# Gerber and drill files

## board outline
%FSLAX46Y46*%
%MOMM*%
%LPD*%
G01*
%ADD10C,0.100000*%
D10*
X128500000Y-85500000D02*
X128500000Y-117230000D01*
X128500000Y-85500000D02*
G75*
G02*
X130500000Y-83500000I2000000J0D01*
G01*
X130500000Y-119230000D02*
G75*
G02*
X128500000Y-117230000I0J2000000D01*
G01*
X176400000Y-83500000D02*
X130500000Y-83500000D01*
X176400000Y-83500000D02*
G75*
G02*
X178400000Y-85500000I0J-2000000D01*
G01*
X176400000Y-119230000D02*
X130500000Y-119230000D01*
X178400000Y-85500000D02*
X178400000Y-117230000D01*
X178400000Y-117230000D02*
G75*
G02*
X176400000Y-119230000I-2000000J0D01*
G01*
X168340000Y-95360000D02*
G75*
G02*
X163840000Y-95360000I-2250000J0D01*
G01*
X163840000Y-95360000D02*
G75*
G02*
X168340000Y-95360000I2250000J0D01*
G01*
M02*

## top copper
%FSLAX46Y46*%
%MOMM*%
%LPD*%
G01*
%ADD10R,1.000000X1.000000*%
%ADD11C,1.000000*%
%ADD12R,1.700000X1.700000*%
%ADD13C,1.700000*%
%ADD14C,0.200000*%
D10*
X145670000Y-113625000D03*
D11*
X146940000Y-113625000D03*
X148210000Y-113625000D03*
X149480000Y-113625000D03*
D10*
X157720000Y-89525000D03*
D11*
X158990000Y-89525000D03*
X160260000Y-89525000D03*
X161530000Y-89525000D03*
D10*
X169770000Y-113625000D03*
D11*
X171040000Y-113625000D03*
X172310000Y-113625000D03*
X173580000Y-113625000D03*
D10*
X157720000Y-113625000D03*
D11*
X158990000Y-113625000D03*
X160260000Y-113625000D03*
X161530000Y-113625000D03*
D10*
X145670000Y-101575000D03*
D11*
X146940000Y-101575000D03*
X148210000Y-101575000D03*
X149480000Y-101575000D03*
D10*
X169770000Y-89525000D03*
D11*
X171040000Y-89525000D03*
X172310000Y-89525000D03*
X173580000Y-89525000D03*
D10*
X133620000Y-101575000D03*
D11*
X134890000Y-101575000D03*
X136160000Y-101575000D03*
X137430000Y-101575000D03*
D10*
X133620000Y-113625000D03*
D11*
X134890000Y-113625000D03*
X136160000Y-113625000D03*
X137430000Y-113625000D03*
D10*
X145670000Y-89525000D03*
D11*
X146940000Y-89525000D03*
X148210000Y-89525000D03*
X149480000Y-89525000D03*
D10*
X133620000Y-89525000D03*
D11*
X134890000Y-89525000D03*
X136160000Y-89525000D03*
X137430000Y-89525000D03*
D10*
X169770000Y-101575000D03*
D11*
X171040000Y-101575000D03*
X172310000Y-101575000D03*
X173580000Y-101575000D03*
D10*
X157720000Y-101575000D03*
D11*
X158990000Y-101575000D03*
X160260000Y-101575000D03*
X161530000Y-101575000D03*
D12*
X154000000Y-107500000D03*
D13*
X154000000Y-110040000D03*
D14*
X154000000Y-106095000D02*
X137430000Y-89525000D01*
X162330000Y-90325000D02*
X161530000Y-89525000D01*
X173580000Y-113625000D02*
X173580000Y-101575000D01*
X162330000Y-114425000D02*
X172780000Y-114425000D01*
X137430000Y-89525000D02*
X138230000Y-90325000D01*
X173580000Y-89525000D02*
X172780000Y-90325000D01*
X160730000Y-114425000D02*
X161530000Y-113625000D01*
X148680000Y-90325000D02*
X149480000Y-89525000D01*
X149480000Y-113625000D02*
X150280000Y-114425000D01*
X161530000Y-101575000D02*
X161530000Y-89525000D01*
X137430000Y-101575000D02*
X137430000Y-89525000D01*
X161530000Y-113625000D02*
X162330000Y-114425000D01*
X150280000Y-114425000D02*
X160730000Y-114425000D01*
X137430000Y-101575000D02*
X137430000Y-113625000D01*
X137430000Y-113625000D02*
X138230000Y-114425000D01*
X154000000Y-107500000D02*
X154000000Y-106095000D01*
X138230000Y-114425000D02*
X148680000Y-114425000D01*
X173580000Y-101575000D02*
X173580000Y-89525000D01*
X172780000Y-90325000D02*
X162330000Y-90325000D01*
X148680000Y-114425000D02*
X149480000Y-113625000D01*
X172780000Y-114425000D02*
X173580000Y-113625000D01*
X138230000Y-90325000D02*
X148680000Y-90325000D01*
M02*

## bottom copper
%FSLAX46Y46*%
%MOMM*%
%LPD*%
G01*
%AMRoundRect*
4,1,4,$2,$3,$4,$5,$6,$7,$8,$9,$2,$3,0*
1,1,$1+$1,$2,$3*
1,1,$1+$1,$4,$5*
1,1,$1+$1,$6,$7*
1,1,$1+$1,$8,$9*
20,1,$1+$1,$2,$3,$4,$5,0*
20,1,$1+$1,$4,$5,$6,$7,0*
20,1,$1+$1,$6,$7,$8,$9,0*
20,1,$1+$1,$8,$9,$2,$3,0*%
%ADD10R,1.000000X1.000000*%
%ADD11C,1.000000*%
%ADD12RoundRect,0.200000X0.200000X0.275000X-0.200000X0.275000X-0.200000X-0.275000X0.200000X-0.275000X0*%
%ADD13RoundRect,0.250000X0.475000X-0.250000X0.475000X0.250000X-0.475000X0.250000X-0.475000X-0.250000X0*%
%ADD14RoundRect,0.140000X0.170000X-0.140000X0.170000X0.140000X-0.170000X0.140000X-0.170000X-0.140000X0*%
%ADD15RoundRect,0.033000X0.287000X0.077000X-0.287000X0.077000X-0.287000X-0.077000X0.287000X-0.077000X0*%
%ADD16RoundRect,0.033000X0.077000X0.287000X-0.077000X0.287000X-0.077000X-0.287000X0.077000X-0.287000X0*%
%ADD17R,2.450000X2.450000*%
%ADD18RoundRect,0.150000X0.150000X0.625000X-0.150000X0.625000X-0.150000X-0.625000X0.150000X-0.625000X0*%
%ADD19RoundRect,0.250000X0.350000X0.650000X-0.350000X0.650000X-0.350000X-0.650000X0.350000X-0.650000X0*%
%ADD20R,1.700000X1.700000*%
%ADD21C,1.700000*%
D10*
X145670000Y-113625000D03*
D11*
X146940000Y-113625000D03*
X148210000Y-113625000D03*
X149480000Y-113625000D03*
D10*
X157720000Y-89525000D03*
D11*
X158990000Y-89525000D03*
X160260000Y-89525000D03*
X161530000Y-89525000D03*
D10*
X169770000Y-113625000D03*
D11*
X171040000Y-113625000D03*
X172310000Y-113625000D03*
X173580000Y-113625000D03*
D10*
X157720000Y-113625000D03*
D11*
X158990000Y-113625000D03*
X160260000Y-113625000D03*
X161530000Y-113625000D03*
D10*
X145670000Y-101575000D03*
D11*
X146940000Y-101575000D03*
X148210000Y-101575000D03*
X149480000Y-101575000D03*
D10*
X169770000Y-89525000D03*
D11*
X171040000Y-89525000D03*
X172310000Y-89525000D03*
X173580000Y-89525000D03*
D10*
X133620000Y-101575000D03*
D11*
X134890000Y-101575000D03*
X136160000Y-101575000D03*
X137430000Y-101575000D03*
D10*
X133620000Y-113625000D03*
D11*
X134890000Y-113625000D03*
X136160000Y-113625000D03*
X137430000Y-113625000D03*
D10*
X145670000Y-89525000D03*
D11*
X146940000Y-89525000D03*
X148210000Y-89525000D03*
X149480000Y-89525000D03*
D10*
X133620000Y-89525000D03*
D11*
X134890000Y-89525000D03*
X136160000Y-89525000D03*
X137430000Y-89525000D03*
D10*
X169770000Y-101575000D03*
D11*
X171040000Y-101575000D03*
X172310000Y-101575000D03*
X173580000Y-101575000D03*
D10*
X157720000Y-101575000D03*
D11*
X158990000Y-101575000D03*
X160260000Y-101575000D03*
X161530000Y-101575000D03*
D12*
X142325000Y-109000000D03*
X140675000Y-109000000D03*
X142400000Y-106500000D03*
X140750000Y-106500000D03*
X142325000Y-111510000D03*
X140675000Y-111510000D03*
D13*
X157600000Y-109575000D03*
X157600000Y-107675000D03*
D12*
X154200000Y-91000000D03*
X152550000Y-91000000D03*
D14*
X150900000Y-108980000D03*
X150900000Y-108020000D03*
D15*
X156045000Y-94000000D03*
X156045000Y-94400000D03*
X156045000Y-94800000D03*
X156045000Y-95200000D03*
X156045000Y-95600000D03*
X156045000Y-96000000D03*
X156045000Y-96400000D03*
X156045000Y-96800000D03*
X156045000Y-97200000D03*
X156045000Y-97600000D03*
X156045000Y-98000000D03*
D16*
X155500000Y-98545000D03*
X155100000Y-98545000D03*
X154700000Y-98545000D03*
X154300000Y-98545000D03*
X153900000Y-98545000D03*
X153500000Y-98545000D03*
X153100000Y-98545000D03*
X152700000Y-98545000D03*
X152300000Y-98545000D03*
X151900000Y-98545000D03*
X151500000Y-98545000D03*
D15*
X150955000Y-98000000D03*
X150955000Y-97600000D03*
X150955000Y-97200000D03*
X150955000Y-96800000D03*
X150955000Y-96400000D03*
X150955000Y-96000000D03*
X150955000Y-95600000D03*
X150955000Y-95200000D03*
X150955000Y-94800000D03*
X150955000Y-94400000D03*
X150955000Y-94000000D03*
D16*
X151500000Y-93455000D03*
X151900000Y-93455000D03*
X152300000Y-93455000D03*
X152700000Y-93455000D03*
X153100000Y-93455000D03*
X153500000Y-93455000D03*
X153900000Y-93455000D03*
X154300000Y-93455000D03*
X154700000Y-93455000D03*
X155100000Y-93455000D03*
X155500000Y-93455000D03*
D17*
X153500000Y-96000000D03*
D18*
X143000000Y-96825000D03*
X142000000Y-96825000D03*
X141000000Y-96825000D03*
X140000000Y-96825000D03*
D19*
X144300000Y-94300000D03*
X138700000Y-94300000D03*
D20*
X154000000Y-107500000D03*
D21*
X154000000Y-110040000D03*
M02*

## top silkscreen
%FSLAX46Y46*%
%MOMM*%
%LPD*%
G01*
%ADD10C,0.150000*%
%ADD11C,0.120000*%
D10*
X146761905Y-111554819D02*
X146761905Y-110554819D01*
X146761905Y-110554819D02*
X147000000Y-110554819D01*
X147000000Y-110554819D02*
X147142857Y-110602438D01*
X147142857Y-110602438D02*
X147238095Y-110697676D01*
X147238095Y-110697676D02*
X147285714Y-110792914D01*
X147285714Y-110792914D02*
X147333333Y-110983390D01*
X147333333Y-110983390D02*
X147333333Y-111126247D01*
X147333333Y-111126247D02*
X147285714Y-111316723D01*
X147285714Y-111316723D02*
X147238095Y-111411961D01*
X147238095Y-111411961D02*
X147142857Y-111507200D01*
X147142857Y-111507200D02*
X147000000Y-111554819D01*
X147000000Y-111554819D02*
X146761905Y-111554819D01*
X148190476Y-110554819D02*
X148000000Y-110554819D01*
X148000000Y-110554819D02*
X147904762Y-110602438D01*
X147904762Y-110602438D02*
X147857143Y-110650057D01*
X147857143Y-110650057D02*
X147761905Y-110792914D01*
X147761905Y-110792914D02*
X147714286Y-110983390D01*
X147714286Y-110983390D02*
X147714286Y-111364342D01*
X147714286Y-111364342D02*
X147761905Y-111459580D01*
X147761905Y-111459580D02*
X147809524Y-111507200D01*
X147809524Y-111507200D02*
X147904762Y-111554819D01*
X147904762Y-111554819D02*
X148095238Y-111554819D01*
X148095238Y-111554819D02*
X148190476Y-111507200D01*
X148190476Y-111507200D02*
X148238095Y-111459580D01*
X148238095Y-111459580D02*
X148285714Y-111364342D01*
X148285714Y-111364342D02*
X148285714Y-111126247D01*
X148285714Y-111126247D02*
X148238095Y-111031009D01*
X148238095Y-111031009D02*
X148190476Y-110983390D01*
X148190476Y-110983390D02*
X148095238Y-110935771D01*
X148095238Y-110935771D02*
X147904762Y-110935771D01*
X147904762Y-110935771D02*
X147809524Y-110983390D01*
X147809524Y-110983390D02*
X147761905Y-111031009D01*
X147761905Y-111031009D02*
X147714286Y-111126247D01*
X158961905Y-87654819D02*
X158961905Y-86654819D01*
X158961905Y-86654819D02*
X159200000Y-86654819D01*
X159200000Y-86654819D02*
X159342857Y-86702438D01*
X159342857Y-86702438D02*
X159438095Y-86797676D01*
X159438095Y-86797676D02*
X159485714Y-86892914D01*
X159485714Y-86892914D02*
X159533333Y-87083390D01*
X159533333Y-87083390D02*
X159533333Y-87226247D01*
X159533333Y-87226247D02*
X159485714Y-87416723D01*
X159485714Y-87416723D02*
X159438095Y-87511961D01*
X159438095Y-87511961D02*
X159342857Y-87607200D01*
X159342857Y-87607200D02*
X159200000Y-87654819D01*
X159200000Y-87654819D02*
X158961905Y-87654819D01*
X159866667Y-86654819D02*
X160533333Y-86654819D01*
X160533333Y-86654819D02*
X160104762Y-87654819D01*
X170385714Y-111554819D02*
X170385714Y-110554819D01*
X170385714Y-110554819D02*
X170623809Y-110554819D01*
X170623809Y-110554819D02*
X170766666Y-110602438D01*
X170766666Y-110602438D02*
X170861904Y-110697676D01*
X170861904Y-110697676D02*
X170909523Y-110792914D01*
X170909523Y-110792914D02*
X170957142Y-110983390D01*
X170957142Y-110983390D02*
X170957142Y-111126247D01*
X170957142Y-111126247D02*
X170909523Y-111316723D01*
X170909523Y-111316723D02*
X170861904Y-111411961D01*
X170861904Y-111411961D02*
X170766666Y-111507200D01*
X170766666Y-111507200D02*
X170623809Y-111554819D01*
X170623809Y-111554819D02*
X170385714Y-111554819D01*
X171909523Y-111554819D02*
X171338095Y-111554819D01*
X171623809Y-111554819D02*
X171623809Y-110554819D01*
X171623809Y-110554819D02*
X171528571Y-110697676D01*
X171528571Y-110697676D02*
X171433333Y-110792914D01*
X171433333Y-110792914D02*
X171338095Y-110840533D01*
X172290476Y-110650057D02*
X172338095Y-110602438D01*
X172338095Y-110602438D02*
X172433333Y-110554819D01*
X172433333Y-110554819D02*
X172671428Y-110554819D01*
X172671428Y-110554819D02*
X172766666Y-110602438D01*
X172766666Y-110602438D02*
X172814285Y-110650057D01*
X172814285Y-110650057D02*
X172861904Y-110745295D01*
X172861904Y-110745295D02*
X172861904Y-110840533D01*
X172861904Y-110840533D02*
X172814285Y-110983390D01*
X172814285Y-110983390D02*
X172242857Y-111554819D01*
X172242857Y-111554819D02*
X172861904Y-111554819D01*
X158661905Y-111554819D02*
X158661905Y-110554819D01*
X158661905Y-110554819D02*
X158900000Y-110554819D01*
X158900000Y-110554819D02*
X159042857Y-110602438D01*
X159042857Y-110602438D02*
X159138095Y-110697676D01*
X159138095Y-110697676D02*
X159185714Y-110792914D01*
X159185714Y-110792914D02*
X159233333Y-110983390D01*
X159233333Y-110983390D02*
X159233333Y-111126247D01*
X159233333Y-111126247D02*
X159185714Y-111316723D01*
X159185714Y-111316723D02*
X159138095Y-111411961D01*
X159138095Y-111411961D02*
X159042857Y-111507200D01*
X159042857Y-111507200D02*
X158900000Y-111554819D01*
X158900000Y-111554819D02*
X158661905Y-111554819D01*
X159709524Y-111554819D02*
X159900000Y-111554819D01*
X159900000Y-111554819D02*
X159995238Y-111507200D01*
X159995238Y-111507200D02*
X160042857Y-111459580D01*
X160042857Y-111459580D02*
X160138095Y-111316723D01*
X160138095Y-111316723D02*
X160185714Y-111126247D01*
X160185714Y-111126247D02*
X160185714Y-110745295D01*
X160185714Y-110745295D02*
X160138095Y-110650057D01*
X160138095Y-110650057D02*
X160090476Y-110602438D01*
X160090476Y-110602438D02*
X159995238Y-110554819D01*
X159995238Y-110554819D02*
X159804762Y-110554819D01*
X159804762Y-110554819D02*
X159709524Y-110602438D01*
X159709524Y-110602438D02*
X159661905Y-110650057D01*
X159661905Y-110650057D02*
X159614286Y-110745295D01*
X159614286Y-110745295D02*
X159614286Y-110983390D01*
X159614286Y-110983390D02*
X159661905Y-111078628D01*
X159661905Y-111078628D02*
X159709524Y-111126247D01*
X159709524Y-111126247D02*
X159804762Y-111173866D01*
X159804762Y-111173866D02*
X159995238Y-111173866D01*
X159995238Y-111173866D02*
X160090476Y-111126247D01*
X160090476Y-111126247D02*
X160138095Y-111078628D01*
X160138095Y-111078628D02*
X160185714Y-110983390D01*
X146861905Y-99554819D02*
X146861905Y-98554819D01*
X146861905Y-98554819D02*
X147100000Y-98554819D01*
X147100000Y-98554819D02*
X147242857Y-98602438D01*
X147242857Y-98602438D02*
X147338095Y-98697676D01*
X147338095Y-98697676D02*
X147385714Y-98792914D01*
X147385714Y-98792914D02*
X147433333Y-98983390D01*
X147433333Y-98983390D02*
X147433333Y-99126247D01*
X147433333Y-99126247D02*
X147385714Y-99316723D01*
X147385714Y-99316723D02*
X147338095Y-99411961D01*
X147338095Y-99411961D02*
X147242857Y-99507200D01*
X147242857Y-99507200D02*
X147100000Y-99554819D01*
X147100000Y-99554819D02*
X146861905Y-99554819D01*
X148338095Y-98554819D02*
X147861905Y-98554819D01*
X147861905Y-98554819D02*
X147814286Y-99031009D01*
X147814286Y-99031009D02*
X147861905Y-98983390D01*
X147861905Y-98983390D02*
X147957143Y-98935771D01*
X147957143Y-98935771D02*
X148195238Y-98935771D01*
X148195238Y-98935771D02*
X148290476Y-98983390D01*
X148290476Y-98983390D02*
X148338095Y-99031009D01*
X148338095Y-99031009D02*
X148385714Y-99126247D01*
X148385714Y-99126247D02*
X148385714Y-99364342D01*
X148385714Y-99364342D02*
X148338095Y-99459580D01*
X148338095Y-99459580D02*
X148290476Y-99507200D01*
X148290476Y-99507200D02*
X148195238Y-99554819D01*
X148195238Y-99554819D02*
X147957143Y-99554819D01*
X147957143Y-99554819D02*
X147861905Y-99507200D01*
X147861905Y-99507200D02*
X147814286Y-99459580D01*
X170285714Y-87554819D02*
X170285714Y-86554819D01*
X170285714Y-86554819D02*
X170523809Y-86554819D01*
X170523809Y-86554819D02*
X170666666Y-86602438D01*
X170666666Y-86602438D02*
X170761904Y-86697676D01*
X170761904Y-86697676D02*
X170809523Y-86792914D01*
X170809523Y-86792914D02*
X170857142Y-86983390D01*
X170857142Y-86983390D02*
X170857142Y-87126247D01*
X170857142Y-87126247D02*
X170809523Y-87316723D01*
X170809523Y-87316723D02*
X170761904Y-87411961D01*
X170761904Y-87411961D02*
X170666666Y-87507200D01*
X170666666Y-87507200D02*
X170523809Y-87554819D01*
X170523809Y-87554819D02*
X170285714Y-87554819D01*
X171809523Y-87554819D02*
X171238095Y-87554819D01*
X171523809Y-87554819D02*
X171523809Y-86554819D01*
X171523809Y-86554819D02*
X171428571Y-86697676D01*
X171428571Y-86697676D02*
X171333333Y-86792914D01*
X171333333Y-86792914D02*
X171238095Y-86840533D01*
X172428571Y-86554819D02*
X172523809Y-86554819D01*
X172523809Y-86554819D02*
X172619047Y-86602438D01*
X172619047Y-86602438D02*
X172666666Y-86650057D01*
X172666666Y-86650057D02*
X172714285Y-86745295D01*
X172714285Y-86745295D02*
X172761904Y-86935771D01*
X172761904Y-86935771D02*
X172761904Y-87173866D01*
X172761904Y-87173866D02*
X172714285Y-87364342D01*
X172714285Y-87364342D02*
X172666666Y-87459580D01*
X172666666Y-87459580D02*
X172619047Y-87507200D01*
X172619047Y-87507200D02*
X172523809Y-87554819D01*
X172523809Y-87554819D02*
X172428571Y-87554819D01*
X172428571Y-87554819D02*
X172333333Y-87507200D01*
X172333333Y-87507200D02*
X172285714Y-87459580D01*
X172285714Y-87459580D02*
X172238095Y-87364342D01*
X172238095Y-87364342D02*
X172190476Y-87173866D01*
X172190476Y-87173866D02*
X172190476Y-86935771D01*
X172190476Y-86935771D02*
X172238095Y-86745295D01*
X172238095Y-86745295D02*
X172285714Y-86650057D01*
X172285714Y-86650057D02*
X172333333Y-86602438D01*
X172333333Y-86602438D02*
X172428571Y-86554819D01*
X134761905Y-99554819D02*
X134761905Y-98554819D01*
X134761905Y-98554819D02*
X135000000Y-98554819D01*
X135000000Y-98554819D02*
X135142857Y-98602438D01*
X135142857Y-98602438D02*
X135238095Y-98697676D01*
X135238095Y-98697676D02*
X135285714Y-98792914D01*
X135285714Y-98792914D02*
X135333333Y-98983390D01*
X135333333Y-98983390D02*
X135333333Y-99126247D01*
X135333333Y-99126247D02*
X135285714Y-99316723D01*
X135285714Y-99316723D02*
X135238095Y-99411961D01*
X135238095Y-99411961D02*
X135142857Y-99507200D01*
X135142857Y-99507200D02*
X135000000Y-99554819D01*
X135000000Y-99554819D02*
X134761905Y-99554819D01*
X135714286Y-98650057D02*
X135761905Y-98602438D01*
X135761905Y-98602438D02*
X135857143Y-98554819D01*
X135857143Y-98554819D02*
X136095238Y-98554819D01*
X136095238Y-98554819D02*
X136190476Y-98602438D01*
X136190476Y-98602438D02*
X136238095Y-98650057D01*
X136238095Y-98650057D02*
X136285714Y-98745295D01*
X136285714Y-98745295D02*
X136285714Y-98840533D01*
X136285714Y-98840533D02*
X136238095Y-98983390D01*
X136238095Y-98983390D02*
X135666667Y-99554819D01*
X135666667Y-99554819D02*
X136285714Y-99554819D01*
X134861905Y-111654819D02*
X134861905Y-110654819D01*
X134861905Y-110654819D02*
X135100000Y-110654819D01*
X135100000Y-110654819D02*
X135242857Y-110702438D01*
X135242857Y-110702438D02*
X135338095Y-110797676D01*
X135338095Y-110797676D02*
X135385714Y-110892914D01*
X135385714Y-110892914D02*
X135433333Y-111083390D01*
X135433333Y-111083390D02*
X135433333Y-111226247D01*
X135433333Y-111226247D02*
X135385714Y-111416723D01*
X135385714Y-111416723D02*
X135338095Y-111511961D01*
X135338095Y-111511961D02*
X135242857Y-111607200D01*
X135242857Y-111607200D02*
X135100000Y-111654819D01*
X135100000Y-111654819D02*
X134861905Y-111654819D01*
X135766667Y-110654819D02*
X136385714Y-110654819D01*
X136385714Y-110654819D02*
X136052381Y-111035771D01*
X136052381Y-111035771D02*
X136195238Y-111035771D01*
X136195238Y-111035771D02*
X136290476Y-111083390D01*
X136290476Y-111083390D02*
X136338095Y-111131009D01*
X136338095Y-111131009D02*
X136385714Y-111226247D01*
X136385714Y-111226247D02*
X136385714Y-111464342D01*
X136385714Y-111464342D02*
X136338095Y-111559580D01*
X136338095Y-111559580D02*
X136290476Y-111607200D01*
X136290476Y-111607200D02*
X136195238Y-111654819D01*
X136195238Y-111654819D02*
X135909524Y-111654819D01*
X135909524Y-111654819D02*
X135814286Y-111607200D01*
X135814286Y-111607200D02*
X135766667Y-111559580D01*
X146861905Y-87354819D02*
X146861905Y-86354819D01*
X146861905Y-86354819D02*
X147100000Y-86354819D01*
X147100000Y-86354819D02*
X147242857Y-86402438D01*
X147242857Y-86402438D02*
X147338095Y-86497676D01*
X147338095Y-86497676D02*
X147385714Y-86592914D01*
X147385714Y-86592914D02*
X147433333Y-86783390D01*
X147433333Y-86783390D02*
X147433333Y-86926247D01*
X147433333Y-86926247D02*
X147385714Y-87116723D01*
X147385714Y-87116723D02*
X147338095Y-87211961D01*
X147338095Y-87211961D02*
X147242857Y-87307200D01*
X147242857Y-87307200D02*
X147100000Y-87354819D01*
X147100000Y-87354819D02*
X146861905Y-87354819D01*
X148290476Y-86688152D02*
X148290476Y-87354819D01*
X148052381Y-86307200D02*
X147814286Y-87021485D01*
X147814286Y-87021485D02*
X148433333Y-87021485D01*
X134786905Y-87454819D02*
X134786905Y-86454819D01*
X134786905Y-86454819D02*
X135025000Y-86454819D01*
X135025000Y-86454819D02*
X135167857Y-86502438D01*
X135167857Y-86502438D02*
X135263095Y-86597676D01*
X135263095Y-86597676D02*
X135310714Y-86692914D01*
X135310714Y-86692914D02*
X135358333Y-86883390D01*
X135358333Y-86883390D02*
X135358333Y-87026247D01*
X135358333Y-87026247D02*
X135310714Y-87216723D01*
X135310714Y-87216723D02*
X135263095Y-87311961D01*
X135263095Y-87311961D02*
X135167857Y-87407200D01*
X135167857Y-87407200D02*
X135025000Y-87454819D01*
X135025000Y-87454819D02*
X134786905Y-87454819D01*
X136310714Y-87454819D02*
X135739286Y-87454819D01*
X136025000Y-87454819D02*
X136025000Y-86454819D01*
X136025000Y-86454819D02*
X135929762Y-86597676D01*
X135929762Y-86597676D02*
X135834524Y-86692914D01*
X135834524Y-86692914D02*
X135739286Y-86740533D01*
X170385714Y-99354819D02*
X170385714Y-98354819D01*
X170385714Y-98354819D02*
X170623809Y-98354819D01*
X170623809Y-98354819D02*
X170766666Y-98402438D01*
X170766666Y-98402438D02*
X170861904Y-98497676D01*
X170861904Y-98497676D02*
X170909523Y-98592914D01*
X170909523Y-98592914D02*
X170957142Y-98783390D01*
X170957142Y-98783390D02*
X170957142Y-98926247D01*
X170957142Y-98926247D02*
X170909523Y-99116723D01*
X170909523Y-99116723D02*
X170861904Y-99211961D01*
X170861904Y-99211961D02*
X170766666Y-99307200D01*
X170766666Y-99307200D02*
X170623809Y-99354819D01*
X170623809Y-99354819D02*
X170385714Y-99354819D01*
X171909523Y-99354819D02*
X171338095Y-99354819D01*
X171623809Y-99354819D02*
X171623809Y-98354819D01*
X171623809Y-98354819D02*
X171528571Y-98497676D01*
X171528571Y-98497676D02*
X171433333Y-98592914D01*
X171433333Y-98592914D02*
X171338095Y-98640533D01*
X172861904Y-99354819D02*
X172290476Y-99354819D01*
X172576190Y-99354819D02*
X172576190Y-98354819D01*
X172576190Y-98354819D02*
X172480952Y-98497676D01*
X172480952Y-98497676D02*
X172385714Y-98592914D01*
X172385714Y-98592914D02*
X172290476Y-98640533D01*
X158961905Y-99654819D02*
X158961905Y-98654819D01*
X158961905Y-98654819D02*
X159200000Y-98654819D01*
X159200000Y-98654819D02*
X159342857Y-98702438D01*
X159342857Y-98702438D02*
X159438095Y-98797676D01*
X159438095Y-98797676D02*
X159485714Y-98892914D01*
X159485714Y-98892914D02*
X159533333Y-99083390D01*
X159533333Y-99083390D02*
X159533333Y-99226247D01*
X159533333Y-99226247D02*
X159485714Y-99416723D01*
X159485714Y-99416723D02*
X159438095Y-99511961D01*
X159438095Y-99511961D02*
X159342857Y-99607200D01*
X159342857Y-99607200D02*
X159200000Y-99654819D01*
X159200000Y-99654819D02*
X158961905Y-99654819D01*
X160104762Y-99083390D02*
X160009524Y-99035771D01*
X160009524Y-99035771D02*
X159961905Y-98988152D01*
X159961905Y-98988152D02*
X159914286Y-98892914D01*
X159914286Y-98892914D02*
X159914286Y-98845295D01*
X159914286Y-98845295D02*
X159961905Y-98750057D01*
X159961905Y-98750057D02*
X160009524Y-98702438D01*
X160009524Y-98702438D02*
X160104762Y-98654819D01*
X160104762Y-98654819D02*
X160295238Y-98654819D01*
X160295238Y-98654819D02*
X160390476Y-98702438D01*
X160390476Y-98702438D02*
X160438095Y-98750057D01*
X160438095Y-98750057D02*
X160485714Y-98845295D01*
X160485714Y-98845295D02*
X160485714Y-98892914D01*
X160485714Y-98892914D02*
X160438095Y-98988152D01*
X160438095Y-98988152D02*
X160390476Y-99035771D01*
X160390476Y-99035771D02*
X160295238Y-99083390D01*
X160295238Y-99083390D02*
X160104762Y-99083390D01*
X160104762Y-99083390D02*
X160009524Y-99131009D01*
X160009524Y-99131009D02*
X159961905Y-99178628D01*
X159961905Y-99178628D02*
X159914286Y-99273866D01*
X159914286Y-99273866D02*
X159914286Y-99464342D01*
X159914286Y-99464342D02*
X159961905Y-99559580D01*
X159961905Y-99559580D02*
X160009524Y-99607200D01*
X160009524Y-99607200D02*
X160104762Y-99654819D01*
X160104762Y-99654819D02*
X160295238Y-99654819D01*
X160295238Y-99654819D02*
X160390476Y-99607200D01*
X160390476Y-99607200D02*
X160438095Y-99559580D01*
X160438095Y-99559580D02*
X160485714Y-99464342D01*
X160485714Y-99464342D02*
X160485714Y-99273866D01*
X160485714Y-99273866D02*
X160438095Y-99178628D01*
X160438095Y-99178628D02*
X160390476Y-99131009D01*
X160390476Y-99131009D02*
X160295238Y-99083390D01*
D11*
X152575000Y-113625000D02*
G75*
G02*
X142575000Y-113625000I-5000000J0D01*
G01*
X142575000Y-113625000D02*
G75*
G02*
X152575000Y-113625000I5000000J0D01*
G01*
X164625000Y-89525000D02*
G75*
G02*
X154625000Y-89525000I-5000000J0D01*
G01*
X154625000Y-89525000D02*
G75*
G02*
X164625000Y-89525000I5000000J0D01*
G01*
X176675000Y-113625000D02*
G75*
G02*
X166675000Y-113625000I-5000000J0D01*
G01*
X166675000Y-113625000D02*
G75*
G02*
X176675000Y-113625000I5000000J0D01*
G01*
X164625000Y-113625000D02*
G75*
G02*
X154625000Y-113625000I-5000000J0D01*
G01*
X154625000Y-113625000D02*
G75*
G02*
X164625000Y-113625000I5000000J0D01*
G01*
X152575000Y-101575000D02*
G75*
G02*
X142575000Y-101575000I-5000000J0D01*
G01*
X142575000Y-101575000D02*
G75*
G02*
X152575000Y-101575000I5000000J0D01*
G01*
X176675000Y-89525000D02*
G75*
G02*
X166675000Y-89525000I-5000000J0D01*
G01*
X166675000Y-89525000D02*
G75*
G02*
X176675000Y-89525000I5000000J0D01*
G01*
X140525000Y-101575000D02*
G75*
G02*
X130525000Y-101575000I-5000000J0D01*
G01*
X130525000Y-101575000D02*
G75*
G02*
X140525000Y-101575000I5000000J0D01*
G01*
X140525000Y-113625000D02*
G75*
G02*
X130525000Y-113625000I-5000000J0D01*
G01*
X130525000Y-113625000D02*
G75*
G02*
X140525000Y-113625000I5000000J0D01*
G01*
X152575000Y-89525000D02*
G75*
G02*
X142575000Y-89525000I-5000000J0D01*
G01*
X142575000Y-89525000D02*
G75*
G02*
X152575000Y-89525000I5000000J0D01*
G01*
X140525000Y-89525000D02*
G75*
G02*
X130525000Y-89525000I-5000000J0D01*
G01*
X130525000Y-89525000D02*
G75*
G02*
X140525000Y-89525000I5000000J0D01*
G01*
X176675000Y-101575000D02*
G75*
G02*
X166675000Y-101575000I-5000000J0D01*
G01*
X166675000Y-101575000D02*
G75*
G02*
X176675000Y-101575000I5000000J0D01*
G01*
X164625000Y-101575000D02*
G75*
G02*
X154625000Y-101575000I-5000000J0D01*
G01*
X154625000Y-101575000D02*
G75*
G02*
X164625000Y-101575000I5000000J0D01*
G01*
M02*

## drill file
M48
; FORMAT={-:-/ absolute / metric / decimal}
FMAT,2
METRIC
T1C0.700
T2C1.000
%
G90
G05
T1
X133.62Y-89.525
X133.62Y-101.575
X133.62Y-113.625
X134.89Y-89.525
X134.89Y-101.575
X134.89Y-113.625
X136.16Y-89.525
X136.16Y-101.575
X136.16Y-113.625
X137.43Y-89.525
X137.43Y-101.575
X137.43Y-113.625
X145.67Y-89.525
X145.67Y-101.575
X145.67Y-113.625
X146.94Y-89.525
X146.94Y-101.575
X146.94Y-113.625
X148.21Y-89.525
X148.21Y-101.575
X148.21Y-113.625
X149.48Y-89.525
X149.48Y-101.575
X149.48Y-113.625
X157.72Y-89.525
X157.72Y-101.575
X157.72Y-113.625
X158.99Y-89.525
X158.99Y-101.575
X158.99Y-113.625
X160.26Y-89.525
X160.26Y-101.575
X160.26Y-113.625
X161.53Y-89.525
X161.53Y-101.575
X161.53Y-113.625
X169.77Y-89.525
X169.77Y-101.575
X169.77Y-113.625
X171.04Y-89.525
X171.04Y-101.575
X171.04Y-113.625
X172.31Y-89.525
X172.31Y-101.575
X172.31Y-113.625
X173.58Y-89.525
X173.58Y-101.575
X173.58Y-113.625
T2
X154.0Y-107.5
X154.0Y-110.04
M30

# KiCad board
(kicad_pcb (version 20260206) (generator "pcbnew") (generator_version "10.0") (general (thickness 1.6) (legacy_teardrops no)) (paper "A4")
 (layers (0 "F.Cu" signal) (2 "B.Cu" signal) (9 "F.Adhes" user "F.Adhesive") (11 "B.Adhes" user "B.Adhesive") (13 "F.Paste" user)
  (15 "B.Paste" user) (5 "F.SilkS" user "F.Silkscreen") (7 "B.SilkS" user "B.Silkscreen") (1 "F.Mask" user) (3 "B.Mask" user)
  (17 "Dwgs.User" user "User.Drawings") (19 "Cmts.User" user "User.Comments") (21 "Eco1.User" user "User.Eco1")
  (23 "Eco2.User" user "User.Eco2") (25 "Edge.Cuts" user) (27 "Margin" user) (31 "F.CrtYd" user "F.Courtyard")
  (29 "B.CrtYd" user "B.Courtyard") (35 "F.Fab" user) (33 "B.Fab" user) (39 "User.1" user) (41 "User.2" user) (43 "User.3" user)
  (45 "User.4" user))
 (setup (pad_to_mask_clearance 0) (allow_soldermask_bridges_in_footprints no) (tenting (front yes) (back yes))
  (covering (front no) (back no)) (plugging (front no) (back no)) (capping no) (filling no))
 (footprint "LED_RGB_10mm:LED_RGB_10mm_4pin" (layer "F.Cu") (at 147.575 113.625)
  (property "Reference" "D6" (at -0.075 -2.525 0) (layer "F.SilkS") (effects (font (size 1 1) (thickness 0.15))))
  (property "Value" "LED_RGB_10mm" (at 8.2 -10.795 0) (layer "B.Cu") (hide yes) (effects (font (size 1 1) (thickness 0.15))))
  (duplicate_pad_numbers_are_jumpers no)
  (fp_circle (center 0 0) (end 5 0) (stroke (width 0.12) (type solid)) (fill no) (layer "F.SilkS"))
  (pad "1" thru_hole rect (at -1.905 0) (size 1 1) (drill 0.7) (layers "*.Cu" "*.Mask") (remove_unused_layers no) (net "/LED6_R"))
  (pad "2" thru_hole circle (at -0.635 0) (size 1 1) (drill 0.7) (layers "*.Cu" "*.Mask") (remove_unused_layers no) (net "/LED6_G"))
  (pad "3" thru_hole circle (at 0.635 0) (size 1 1) (drill 0.7) (layers "*.Cu" "*.Mask") (remove_unused_layers no) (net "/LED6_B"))
  (pad "4" thru_hole circle (at 1.905 0) (size 1 1) (drill 0.7) (layers "*.Cu" "*.Mask") (remove_unused_layers no) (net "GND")))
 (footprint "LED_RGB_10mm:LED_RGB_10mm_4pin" (layer "F.Cu") (at 159.625 89.525)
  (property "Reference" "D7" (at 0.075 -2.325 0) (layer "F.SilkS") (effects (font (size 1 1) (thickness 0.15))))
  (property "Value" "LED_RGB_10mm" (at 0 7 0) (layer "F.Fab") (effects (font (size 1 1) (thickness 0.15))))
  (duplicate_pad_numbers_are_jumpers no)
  (fp_circle (center 0 0) (end 5 0) (stroke (width 0.12) (type solid)) (fill no) (layer "F.SilkS"))
  (pad "1" thru_hole rect (at -1.905 0) (size 1 1) (drill 0.7) (layers "*.Cu" "*.Mask") (remove_unused_layers no) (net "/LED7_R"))
  (pad "2" thru_hole circle (at -0.635 0) (size 1 1) (drill 0.7) (layers "*.Cu" "*.Mask") (remove_unused_layers no) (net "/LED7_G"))
  (pad "3" thru_hole circle (at 0.635 0) (size 1 1) (drill 0.7) (layers "*.Cu" "*.Mask") (remove_unused_layers no) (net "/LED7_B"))
  (pad "4" thru_hole circle (at 1.905 0) (size 1 1) (drill 0.7) (layers "*.Cu" "*.Mask") (remove_unused_layers no) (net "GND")))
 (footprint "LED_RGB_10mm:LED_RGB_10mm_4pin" (layer "F.Cu") (at 171.675 113.625)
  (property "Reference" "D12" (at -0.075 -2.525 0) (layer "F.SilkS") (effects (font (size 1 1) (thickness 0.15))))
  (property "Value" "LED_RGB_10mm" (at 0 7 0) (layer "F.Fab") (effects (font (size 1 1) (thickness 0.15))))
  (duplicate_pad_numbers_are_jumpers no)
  (fp_circle (center 0 0) (end 5 0) (stroke (width 0.12) (type solid)) (fill no) (layer "F.SilkS"))
  (pad "1" thru_hole rect (at -1.905 0) (size 1 1) (drill 0.7) (layers "*.Cu" "*.Mask") (remove_unused_layers no) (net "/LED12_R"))
  (pad "2" thru_hole circle (at -0.635 0) (size 1 1) (drill 0.7) (layers "*.Cu" "*.Mask") (remove_unused_layers no) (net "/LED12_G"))
  (pad "3" thru_hole circle (at 0.635 0) (size 1 1) (drill 0.7) (layers "*.Cu" "*.Mask") (remove_unused_layers no) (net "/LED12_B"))
  (pad "4" thru_hole circle (at 1.905 0) (size 1 1) (drill 0.7) (layers "*.Cu" "*.Mask") (remove_unused_layers no) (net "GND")))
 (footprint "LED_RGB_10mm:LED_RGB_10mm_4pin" (layer "F.Cu") (at 159.625 113.625)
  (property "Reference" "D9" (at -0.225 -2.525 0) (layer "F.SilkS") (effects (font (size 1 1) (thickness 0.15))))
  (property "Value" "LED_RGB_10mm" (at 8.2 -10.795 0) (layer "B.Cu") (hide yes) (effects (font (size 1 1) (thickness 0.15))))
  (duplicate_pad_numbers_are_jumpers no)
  (fp_circle (center 0 0) (end 5 0) (stroke (width 0.12) (type solid)) (fill no) (layer "F.SilkS"))
  (pad "1" thru_hole rect (at -1.905 0) (size 1 1) (drill 0.7) (layers "*.Cu" "*.Mask") (remove_unused_layers no) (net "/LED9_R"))
  (pad "2" thru_hole circle (at -0.635 0) (size 1 1) (drill 0.7) (layers "*.Cu" "*.Mask") (remove_unused_layers no) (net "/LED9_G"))
  (pad "3" thru_hole circle (at 0.635 0) (size 1 1) (drill 0.7) (layers "*.Cu" "*.Mask") (remove_unused_layers no) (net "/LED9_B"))
  (pad "4" thru_hole circle (at 1.905 0) (size 1 1) (drill 0.7) (layers "*.Cu" "*.Mask") (remove_unused_layers no) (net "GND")))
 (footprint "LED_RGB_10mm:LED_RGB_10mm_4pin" (layer "F.Cu") (at 147.575 101.575)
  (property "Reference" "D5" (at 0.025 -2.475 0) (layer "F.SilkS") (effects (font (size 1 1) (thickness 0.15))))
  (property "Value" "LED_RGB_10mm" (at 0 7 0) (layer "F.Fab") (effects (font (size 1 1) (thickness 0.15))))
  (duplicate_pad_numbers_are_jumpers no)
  (fp_circle (center 0 0) (end 5 0) (stroke (width 0.12) (type solid)) (fill no) (layer "F.SilkS"))
  (pad "1" thru_hole rect (at -1.905 0) (size 1 1) (drill 0.7) (layers "*.Cu" "*.Mask") (remove_unused_layers no) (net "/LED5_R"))
  (pad "2" thru_hole circle (at -0.635 0) (size 1 1) (drill 0.7) (layers "*.Cu" "*.Mask") (remove_unused_layers no) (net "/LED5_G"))
  (pad "3" thru_hole circle (at 0.635 0) (size 1 1) (drill 0.7) (layers "*.Cu" "*.Mask") (remove_unused_layers no) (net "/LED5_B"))
  (pad "4" thru_hole circle (at 1.905 0) (size 1 1) (drill 0.7) (layers "*.Cu" "*.Mask") (remove_unused_layers no) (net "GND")))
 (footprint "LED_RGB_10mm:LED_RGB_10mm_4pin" (layer "F.Cu") (at 171.675 89.525)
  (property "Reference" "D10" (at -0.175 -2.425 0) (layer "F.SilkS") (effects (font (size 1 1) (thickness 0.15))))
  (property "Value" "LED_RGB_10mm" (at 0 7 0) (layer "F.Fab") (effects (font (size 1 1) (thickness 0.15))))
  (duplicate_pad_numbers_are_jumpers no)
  (fp_circle (center 0 0) (end 5 0) (stroke (width 0.12) (type solid)) (fill no) (layer "F.SilkS"))
  (pad "1" thru_hole rect (at -1.905 0) (size 1 1) (drill 0.7) (layers "*.Cu" "*.Mask") (remove_unused_layers no) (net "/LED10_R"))
  (pad "2" thru_hole circle (at -0.635 0) (size 1 1) (drill 0.7) (layers "*.Cu" "*.Mask") (remove_unused_layers no) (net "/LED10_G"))
  (pad "3" thru_hole circle (at 0.635 0) (size 1 1) (drill 0.7) (layers "*.Cu" "*.Mask") (remove_unused_layers no) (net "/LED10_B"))
  (pad "4" thru_hole circle (at 1.905 0) (size 1 1) (drill 0.7) (layers "*.Cu" "*.Mask") (remove_unused_layers no) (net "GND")))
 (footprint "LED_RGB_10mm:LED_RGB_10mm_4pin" (layer "F.Cu") (at 135.525 101.575)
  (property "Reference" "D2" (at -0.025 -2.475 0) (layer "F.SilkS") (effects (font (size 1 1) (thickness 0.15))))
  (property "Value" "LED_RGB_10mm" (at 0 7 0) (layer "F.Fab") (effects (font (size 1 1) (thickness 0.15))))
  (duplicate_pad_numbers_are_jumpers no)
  (fp_circle (center 0 0) (end 5 0) (stroke (width 0.12) (type solid)) (fill no) (layer "F.SilkS"))
  (pad "1" thru_hole rect (at -1.905 0) (size 1 1) (drill 0.7) (layers "*.Cu" "*.Mask") (remove_unused_layers no) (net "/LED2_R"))
  (pad "2" thru_hole circle (at -0.635 0) (size 1 1) (drill 0.7) (layers "*.Cu" "*.Mask") (remove_unused_layers no) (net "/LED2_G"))
  (pad "3" thru_hole circle (at 0.635 0) (size 1 1) (drill 0.7) (layers "*.Cu" "*.Mask") (remove_unused_layers no) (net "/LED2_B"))
  (pad "4" thru_hole circle (at 1.905 0) (size 1 1) (drill 0.7) (layers "*.Cu" "*.Mask") (remove_unused_layers no) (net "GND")))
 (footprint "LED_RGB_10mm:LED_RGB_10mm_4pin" (layer "F.Cu") (at 135.525 113.625)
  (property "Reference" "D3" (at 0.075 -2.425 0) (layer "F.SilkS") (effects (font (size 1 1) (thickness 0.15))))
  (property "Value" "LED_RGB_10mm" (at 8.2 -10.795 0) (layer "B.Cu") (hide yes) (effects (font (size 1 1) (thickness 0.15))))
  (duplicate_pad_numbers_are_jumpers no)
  (fp_circle (center 0 0) (end 5 0) (stroke (width 0.12) (type solid)) (fill no) (layer "F.SilkS"))
  (pad "1" thru_hole rect (at -1.905 0) (size 1 1) (drill 0.7) (layers "*.Cu" "*.Mask") (remove_unused_layers no) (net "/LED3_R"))
  (pad "2" thru_hole circle (at -0.635 0) (size 1 1) (drill 0.7) (layers "*.Cu" "*.Mask") (remove_unused_layers no) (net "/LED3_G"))
  (pad "3" thru_hole circle (at 0.635 0) (size 1 1) (drill 0.7) (layers "*.Cu" "*.Mask") (remove_unused_layers no) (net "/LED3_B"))
  (pad "4" thru_hole circle (at 1.905 0) (size 1 1) (drill 0.7) (layers "*.Cu" "*.Mask") (remove_unused_layers no) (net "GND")))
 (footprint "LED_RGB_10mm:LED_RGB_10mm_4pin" (layer "F.Cu") (at 147.575 89.525)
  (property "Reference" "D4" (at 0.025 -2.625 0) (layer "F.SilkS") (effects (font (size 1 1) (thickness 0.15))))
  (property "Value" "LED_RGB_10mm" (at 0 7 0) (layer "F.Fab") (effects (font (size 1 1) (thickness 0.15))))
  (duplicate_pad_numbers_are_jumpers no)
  (fp_circle (center 0 0) (end 5 0) (stroke (width 0.12) (type solid)) (fill no) (layer "F.SilkS"))
  (pad "1" thru_hole rect (at -1.905 0) (size 1 1) (drill 0.7) (layers "*.Cu" "*.Mask") (remove_unused_layers no) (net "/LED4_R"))
  (pad "2" thru_hole circle (at -0.635 0) (size 1 1) (drill 0.7) (layers "*.Cu" "*.Mask") (remove_unused_layers no) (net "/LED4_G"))
  (pad "3" thru_hole circle (at 0.635 0) (size 1 1) (drill 0.7) (layers "*.Cu" "*.Mask") (remove_unused_layers no) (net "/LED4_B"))
  (pad "4" thru_hole circle (at 1.905 0) (size 1 1) (drill 0.7) (layers "*.Cu" "*.Mask") (remove_unused_layers no) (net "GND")))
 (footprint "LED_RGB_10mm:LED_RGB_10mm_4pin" (layer "F.Cu") (at 135.525 89.525)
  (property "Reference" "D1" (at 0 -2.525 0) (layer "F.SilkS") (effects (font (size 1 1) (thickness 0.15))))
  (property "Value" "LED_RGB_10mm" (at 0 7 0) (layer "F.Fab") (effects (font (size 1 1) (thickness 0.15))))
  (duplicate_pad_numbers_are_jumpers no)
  (fp_circle (center 0 0) (end 5 0) (stroke (width 0.12) (type solid)) (fill no) (layer "F.SilkS"))
  (pad "1" thru_hole rect (at -1.905 0) (size 1 1) (drill 0.7) (layers "*.Cu" "*.Mask") (remove_unused_layers no) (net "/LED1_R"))
  (pad "2" thru_hole circle (at -0.635 0) (size 1 1) (drill 0.7) (layers "*.Cu" "*.Mask") (remove_unused_layers no) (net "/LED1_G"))
  (pad "3" thru_hole circle (at 0.635 0) (size 1 1) (drill 0.7) (layers "*.Cu" "*.Mask") (remove_unused_layers no) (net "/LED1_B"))
  (pad "4" thru_hole circle (at 1.905 0) (size 1 1) (drill 0.7) (layers "*.Cu" "*.Mask") (remove_unused_layers no) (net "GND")))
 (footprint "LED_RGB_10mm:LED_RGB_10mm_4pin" (layer "F.Cu") (at 171.675 101.575)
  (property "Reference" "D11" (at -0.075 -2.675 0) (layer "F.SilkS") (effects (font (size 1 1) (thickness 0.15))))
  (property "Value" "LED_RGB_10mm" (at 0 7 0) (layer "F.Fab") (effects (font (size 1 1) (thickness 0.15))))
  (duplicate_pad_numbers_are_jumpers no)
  (fp_circle (center 0 0) (end 5 0) (stroke (width 0.12) (type solid)) (fill no) (layer "F.SilkS"))
  (pad "1" thru_hole rect (at -1.905 0) (size 1 1) (drill 0.7) (layers "*.Cu" "*.Mask") (remove_unused_layers no) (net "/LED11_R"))
  (pad "2" thru_hole circle (at -0.635 0) (size 1 1) (drill 0.7) (layers "*.Cu" "*.Mask") (remove_unused_layers no) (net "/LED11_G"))
  (pad "3" thru_hole circle (at 0.635 0) (size 1 1) (drill 0.7) (layers "*.Cu" "*.Mask") (remove_unused_layers no) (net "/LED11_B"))
  (pad "4" thru_hole circle (at 1.905 0) (size 1 1) (drill 0.7) (layers "*.Cu" "*.Mask") (remove_unused_layers no) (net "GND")))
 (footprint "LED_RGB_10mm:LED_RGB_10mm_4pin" (layer "F.Cu") (at 159.625 101.575)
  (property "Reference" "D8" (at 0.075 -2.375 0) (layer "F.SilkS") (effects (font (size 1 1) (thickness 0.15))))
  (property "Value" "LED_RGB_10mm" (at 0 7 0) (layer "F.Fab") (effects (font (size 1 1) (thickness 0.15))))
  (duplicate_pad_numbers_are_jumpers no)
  (fp_circle (center 0 0) (end 5 0) (stroke (width 0.12) (type solid)) (fill no) (layer "F.SilkS"))
  (pad "1" thru_hole rect (at -1.905 0) (size 1 1) (drill 0.7) (layers "*.Cu" "*.Mask") (remove_unused_layers no) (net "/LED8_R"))
  (pad "2" thru_hole circle (at -0.635 0) (size 1 1) (drill 0.7) (layers "*.Cu" "*.Mask") (remove_unused_layers no) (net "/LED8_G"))
  (pad "3" thru_hole circle (at 0.635 0) (size 1 1) (drill 0.7) (layers "*.Cu" "*.Mask") (remove_unused_layers no) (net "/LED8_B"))
  (pad "4" thru_hole circle (at 1.905 0) (size 1 1) (drill 0.7) (layers "*.Cu" "*.Mask") (remove_unused_layers no) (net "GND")))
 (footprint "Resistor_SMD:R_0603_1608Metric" (layer "B.Cu") (at 141.5 109 180)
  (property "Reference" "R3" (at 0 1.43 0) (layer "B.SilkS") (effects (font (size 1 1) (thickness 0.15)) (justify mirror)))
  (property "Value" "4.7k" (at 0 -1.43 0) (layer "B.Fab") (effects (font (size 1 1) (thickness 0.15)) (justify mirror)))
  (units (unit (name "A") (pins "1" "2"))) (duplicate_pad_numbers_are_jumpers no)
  (pad "1" smd roundrect (at -0.825 0 180) (size 0.8 0.95) (layers "B.Cu" "B.Mask" "B.Paste") (roundrect_rratio 0.25) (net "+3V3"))
  (pad "2" smd roundrect (at 0.825 0 180) (size 0.8 0.95) (layers "B.Cu" "B.Mask" "B.Paste") (roundrect_rratio 0.25) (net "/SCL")))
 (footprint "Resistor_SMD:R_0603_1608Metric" (layer "B.Cu") (at 141.575 106.5 180)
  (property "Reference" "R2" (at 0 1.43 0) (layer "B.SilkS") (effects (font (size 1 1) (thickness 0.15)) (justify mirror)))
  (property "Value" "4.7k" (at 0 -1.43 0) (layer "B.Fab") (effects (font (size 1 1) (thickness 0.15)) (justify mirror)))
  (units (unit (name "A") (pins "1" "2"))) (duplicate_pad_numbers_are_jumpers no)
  (pad "1" smd roundrect (at -0.825 0 180) (size 0.8 0.95) (layers "B.Cu" "B.Mask" "B.Paste") (roundrect_rratio 0.25) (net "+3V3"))
  (pad "2" smd roundrect (at 0.825 0 180) (size 0.8 0.95) (layers "B.Cu" "B.Mask" "B.Paste") (roundrect_rratio 0.25) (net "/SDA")))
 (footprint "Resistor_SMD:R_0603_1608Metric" (layer "B.Cu") (at 141.5 111.51 180)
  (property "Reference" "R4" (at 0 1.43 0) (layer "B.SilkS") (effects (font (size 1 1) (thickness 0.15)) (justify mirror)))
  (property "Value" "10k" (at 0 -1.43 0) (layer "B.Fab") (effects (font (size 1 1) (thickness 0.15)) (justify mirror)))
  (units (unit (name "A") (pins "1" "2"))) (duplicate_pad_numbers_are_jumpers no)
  (pad "1" smd roundrect (at -0.825 0 180) (size 0.8 0.95) (layers "B.Cu" "B.Mask" "B.Paste") (roundrect_rratio 0.25) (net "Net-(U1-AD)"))
  (pad "2" smd roundrect (at 0.825 0 180) (size 0.8 0.95) (layers "B.Cu" "B.Mask" "B.Paste") (roundrect_rratio 0.25) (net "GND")))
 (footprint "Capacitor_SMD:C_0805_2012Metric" (layer "B.Cu") (at 157.6 108.625 90)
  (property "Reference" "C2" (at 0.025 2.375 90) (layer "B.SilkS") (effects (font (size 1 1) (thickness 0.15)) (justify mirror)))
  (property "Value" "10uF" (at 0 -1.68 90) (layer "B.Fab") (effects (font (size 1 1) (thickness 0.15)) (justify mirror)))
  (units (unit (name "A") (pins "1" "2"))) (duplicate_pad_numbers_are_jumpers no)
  (pad "1" smd roundrect (at -0.95 0 90) (size 1 1.45) (layers "B.Cu" "B.Mask" "B.Paste") (roundrect_rratio 0.25) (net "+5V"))
  (pad "2" smd roundrect (at 0.95 0 90) (size 1 1.45) (layers "B.Cu" "B.Mask" "B.Paste") (roundrect_rratio 0.25) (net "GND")))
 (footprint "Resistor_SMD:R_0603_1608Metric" (layer "B.Cu") (at 153.375 91 180)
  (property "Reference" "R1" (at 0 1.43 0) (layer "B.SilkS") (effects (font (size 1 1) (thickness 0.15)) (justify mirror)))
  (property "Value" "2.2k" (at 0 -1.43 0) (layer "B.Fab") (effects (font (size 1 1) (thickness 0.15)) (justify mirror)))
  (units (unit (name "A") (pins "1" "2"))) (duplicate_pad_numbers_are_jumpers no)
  (pad "1" smd roundrect (at -0.825 0 180) (size 0.8 0.95) (layers "B.Cu" "B.Mask" "B.Paste") (roundrect_rratio 0.25) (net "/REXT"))
  (pad "2" smd roundrect (at 0.825 0 180) (size 0.8 0.95) (layers "B.Cu" "B.Mask" "B.Paste") (roundrect_rratio 0.25) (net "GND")))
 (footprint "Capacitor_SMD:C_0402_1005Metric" (layer "B.Cu") (at 150.9 108.5 90)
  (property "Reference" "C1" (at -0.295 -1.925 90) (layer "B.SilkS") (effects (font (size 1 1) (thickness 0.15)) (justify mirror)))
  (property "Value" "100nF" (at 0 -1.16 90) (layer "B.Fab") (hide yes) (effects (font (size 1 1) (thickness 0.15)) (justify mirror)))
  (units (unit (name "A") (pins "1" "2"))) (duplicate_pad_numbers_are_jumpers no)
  (pad "1" smd roundrect (at -0.48 0 90) (size 0.56 0.62) (layers "B.Cu" "B.Mask" "B.Paste") (roundrect_rratio 0.25) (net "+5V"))
  (pad "2" smd roundrect (at 0.48 0 90) (size 0.56 0.62) (layers "B.Cu" "B.Mask" "B.Paste") (roundrect_rratio 0.25) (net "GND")))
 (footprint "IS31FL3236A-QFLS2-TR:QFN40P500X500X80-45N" (layer "B.Cu") (at 153.5 96 180)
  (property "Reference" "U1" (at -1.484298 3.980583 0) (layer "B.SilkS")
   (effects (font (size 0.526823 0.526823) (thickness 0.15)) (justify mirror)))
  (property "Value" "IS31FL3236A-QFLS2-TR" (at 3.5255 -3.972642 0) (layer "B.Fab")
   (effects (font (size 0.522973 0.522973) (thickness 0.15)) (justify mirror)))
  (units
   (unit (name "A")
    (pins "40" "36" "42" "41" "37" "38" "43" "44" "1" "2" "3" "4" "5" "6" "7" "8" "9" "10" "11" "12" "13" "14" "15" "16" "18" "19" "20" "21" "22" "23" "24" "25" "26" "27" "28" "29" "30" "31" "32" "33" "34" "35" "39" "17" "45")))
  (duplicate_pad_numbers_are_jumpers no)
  (pad "1" smd roundrect (at -2.545 2 180) (size 0.64 0.22) (layers "B.Cu" "B.Mask" "B.Paste") (roundrect_rratio 0.15) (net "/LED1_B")
   (solder_mask_margin 0.102))
  (pad "2" smd roundrect (at -2.545 1.6 180) (size 0.64 0.22) (layers "B.Cu" "B.Mask" "B.Paste") (roundrect_rratio 0.15) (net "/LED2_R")
   (solder_mask_margin 0.102))
  (pad "3" smd roundrect (at -2.545 1.2 180) (size 0.64 0.22) (layers "B.Cu" "B.Mask" "B.Paste") (roundrect_rratio 0.15) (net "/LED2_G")
   (solder_mask_margin 0.102))
  (pad "4" smd roundrect (at -2.545 0.8 180) (size 0.64 0.22) (layers "B.Cu" "B.Mask" "B.Paste") (roundrect_rratio 0.15) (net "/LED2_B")
   (solder_mask_margin 0.102))
  (pad "5" smd roundrect (at -2.545 0.4 180) (size 0.64 0.22) (layers "B.Cu" "B.Mask" "B.Paste") (roundrect_rratio 0.15) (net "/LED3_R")
   (solder_mask_margin 0.102))
  (pad "6" smd roundrect (at -2.545 0 180) (size 0.64 0.22) (layers "B.Cu" "B.Mask" "B.Paste") (roundrect_rratio 0.15) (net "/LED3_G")
   (solder_mask_margin 0.102))
  (pad "7" smd roundrect (at -2.545 -0.4 180) (size 0.64 0.22) (layers "B.Cu" "B.Mask" "B.Paste") (roundrect_rratio 0.15) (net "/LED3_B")
   (solder_mask_margin 0.102))
  (pad "8" smd roundrect (at -2.545 -0.8 180) (size 0.64 0.22) (layers "B.Cu" "B.Mask" "B.Paste") (roundrect_rratio 0.15) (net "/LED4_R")
   (solder_mask_margin 0.102))
  (pad "9" smd roundrect (at -2.545 -1.2 180) (size 0.64 0.22) (layers "B.Cu" "B.Mask" "B.Paste") (roundrect_rratio 0.15) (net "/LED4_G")
   (solder_mask_margin 0.102))
  (pad "10" smd roundrect (at -2.545 -1.6 180) (size 0.64 0.22) (layers "B.Cu" "B.Mask" "B.Paste") (roundrect_rratio 0.15) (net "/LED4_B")
   (solder_mask_margin 0.102))
  (pad "11" smd roundrect (at -2.545 -2 180) (size 0.64 0.22) (layers "B.Cu" "B.Mask" "B.Paste") (roundrect_rratio 0.15) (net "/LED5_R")
   (solder_mask_margin 0.102))
  (pad "12" smd roundrect (at -2 -2.545 180) (size 0.22 0.64) (layers "B.Cu" "B.Mask" "B.Paste") (roundrect_rratio 0.15) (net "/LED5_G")
   (solder_mask_margin 0.102))
  (pad "13" smd roundrect (at -1.6 -2.545 180) (size 0.22 0.64) (layers "B.Cu" "B.Mask" "B.Paste") (roundrect_rratio 0.15) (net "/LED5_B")
   (solder_mask_margin 0.102))
  (pad "14" smd roundrect (at -1.2 -2.545 180) (size 0.22 0.64) (layers "B.Cu" "B.Mask" "B.Paste") (roundrect_rratio 0.15) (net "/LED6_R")
   (solder_mask_margin 0.102))
  (pad "15" smd roundrect (at -0.8 -2.545 180) (size 0.22 0.64) (layers "B.Cu" "B.Mask" "B.Paste") (roundrect_rratio 0.15) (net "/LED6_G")
   (solder_mask_margin 0.102))
  (pad "16" smd roundrect (at -0.4 -2.545 180) (size 0.22 0.64) (layers "B.Cu" "B.Mask" "B.Paste") (roundrect_rratio 0.15) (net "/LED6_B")
   (solder_mask_margin 0.102))
  (pad "17" smd roundrect (at 0 -2.545 180) (size 0.22 0.64) (layers "B.Cu" "B.Mask" "B.Paste") (roundrect_rratio 0.15) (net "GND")
   (solder_mask_margin 0.102))
  (pad "18" smd roundrect (at 0.4 -2.545 180) (size 0.22 0.64) (layers "B.Cu" "B.Mask" "B.Paste") (roundrect_rratio 0.15) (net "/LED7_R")
   (solder_mask_margin 0.102))
  (pad "19" smd roundrect (at 0.8 -2.545 180) (size 0.22 0.64) (layers "B.Cu" "B.Mask" "B.Paste") (roundrect_rratio 0.15) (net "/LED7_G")
   (solder_mask_margin 0.102))
  (pad "20" smd roundrect (at 1.2 -2.545 180) (size 0.22 0.64) (layers "B.Cu" "B.Mask" "B.Paste") (roundrect_rratio 0.15) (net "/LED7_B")
   (solder_mask_margin 0.102))
  (pad "21" smd roundrect (at 1.6 -2.545 180) (size 0.22 0.64) (layers "B.Cu" "B.Mask" "B.Paste") (roundrect_rratio 0.15) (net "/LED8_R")
   (solder_mask_margin 0.102))
  (pad "22" smd roundrect (at 2 -2.545 180) (size 0.22 0.64) (layers "B.Cu" "B.Mask" "B.Paste") (roundrect_rratio 0.15) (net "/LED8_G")
   (solder_mask_margin 0.102))
  (pad "23" smd roundrect (at 2.545 -2 180) (size 0.64 0.22) (layers "B.Cu" "B.Mask" "B.Paste") (roundrect_rratio 0.15) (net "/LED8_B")
   (solder_mask_margin 0.102))
  (pad "24" smd roundrect (at 2.545 -1.6 180) (size 0.64 0.22) (layers "B.Cu" "B.Mask" "B.Paste") (roundrect_rratio 0.15) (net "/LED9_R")
   (solder_mask_margin 0.102))
  (pad "25" smd roundrect (at 2.545 -1.2 180) (size 0.64 0.22) (layers "B.Cu" "B.Mask" "B.Paste") (roundrect_rratio 0.15) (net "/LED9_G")
   (solder_mask_margin 0.102))
  (pad "26" smd roundrect (at 2.545 -0.8 180) (size 0.64 0.22) (layers "B.Cu" "B.Mask" "B.Paste") (roundrect_rratio 0.15) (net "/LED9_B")
   (solder_mask_margin 0.102))
  (pad "27" smd roundrect (at 2.545 -0.4 180) (size 0.64 0.22) (layers "B.Cu" "B.Mask" "B.Paste") (roundrect_rratio 0.15) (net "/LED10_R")
   (solder_mask_margin 0.102))
  (pad "28" smd roundrect (at 2.545 0 180) (size 0.64 0.22) (layers "B.Cu" "B.Mask" "B.Paste") (roundrect_rratio 0.15) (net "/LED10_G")
   (solder_mask_margin 0.102))
  (pad "29" smd roundrect (at 2.545 0.4 180) (size 0.64 0.22) (layers "B.Cu" "B.Mask" "B.Paste") (roundrect_rratio 0.15) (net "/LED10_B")
   (solder_mask_margin 0.102))
  (pad "30" smd roundrect (at 2.545 0.8 180) (size 0.64 0.22) (layers "B.Cu" "B.Mask" "B.Paste") (roundrect_rratio 0.15) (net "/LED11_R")
   (solder_mask_margin 0.102))
  (pad "31" smd roundrect (at 2.545 1.2 180) (size 0.64 0.22) (layers "B.Cu" "B.Mask" "B.Paste") (roundrect_rratio 0.15) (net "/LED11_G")
   (solder_mask_margin 0.102))
  (pad "32" smd roundrect (at 2.545 1.6 180) (size 0.64 0.22) (layers "B.Cu" "B.Mask" "B.Paste") (roundrect_rratio 0.15) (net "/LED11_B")
   (solder_mask_margin 0.102))
  (pad "33" smd roundrect (at 2.545 2 180) (size 0.64 0.22) (layers "B.Cu" "B.Mask" "B.Paste") (roundrect_rratio 0.15) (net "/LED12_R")
   (solder_mask_margin 0.102))
  (pad "34" smd roundrect (at 2 2.545 180) (size 0.22 0.64) (layers "B.Cu" "B.Mask" "B.Paste") (roundrect_rratio 0.15) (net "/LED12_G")
   (solder_mask_margin 0.102))
  (pad "35" smd roundrect (at 1.6 2.545 180) (size 0.22 0.64) (layers "B.Cu" "B.Mask" "B.Paste") (roundrect_rratio 0.15) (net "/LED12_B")
   (solder_mask_margin 0.102))
  (pad "36" smd roundrect (at 1.2 2.545 180) (size 0.22 0.64) (layers "B.Cu" "B.Mask" "B.Paste") (roundrect_rratio 0.15) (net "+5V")
   (solder_mask_margin 0.102))
  (pad "37" smd roundrect (at 0.8 2.545 180) (size 0.22 0.64) (layers "B.Cu" "B.Mask" "B.Paste") (roundrect_rratio 0.15) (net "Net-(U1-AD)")
   (solder_mask_margin 0.102))
  (pad "38" smd roundrect (at 0.4 2.545 180) (size 0.22 0.64) (layers "B.Cu" "B.Mask" "B.Paste") (roundrect_rratio 0.15) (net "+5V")
   (solder_mask_margin 0.102))
  (pad "39" smd roundrect (at 0 2.545 180) (size 0.22 0.64) (layers "B.Cu" "B.Mask" "B.Paste") (roundrect_rratio 0.15) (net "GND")
   (solder_mask_margin 0.102))
  (pad "40" smd roundrect (at -0.4 2.545 180) (size 0.22 0.64) (layers "B.Cu" "B.Mask" "B.Paste") (roundrect_rratio 0.15) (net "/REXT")
   (solder_mask_margin 0.102))
  (pad "41" smd roundrect (at -0.8 2.545 180) (size 0.22 0.64) (layers "B.Cu" "B.Mask" "B.Paste") (roundrect_rratio 0.15) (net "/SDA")
   (solder_mask_margin 0.102))
  (pad "42" smd roundrect (at -1.2 2.545 180) (size 0.22 0.64) (layers "B.Cu" "B.Mask" "B.Paste") (roundrect_rratio 0.15) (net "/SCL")
   (solder_mask_margin 0.102))
  (pad "43" smd roundrect (at -1.6 2.545 180) (size 0.22 0.64) (layers "B.Cu" "B.Mask" "B.Paste") (roundrect_rratio 0.15) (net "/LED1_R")
   (solder_mask_margin 0.102))
  (pad "44" smd roundrect (at -2 2.545 180) (size 0.22 0.64) (layers "B.Cu" "B.Mask" "B.Paste") (roundrect_rratio 0.15) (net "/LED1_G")
   (solder_mask_margin 0.102))
  (pad "45" smd rect (at 0 0 180) (size 2.45 2.45) (layers "B.Cu" "B.Mask") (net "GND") (solder_mask_margin 0.102)))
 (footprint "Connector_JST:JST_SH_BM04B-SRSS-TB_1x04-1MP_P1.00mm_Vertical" (layer "B.Cu") (at 141.5 95.5 180)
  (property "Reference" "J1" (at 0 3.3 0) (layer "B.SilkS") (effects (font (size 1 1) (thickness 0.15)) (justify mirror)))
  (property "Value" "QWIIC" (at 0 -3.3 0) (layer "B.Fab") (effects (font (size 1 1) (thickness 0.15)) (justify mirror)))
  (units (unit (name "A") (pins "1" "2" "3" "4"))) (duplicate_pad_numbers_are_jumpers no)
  (pad "1" smd roundrect (at -1.5 -1.325 180) (size 0.6 1.55) (layers "B.Cu" "B.Mask" "B.Paste") (roundrect_rratio 0.25) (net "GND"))
  (pad "2" smd roundrect (at -0.5 -1.325 180) (size 0.6 1.55) (layers "B.Cu" "B.Mask" "B.Paste") (roundrect_rratio 0.25) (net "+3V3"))
  (pad "3" smd roundrect (at 0.5 -1.325 180) (size 0.6 1.55) (layers "B.Cu" "B.Mask" "B.Paste") (roundrect_rratio 0.25) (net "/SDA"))
  (pad "4" smd roundrect (at 1.5 -1.325 180) (size 0.6 1.55) (layers "B.Cu" "B.Mask" "B.Paste") (roundrect_rratio 0.25) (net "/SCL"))
  (pad "MP" smd roundrect (at -2.8 1.2 180) (size 1.2 1.8) (layers "B.Cu" "B.Mask" "B.Paste") (roundrect_rratio 0.208333))
  (pad "MP" smd roundrect (at 2.8 1.2 180) (size 1.2 1.8) (layers "B.Cu" "B.Mask" "B.Paste") (roundrect_rratio 0.208333)))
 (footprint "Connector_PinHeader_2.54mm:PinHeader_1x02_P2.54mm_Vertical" (layer "B.Cu") (at 154 107.5 180)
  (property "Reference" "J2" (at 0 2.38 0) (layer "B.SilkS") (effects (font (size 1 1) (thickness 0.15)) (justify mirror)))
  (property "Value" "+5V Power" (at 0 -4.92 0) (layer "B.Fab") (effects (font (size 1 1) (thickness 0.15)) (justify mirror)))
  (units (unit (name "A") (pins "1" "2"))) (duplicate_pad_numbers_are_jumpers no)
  (pad "1" thru_hole rect (at 0 0 180) (size 1.7 1.7) (drill 1) (layers "*.Cu" "*.Mask") (remove_unused_layers no) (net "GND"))
  (pad "2" thru_hole circle (at 0 -2.54 180) (size 1.7 1.7) (drill 1) (layers "*.Cu" "*.Mask") (remove_unused_layers no) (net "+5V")))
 (gr_line (start 128.5 85.5) (end 128.5 117.23) (stroke (width 0.1) (type default)) (layer "Edge.Cuts"))
 (gr_arc (start 128.5 85.5) (mid 129.085786 84.085786) (end 130.5 83.5) (stroke (width 0.1) (type default)) (layer "Edge.Cuts"))
 (gr_arc (start 130.5 119.23) (mid 129.085786 118.644214) (end 128.5 117.23) (stroke (width 0.1) (type default)) (layer "Edge.Cuts"))
 (gr_line (start 176.4 83.5) (end 130.5 83.5) (stroke (width 0.1) (type default)) (layer "Edge.Cuts"))
 (gr_arc (start 176.4 83.5) (mid 177.814214 84.085786) (end 178.4 85.5) (stroke (width 0.1) (type default)) (layer "Edge.Cuts"))
 (gr_line (start 176.4 119.23) (end 130.5 119.23) (stroke (width 0.1) (type default)) (layer "Edge.Cuts"))
 (gr_line (start 178.4 85.5) (end 178.4 117.23) (stroke (width 0.1) (type default)) (layer "Edge.Cuts"))
 (gr_arc (start 178.4 117.23) (mid 177.814214 118.644214) (end 176.4 119.23) (stroke (width 0.1) (type default)) (layer "Edge.Cuts"))
 (gr_circle (center 166.09 95.36) (end 168.34 95.36) (stroke (width 0.1) (type default)) (fill none) (layer "Edge.Cuts"))
 (segment (start 154 106.095) (end 137.43 89.525) (width 0.2) (layer "F.Cu") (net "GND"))
 (segment (start 162.33 90.325) (end 161.53 89.525) (width 0.2) (layer "F.Cu") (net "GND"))
 (segment (start 173.58 113.625) (end 173.58 101.575) (width 0.2) (layer "F.Cu") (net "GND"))
 (segment (start 162.33 114.425) (end 172.78 114.425) (width 0.2) (layer "F.Cu") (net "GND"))
 (segment (start 137.43 89.525) (end 138.23 90.325) (width 0.2) (layer "F.Cu") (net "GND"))
 (segment (start 173.58 89.525) (end 172.78 90.325) (width 0.2) (layer "F.Cu") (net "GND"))
 (segment (start 160.73 114.425) (end 161.53 113.625) (width 0.2) (layer "F.Cu") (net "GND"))
 (segment (start 148.68 90.325) (end 149.48 89.525) (width 0.2) (layer "F.Cu") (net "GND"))
 (segment (start 149.48 113.625) (end 150.28 114.425) (width 0.2) (layer "F.Cu") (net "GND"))
 (segment (start 161.53 101.575) (end 161.53 89.525) (width 0.2) (layer "F.Cu") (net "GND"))
 (segment (start 137.43 101.575) (end 137.43 89.525) (width 0.2) (layer "F.Cu") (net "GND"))
 (segment (start 161.53 113.625) (end 162.33 114.425) (width 0.2) (layer "F.Cu") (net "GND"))
 (segment (start 150.28 114.425) (end 160.73 114.425) (width 0.2) (layer "F.Cu") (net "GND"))
 (segment (start 137.43 101.575) (end 137.43 113.625) (width 0.2) (layer "F.Cu") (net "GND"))
 (segment (start 137.43 113.625) (end 138.23 114.425) (width 0.2) (layer "F.Cu") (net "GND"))
 (segment (start 154 107.5) (end 154 106.095) (width 0.2) (layer "F.Cu") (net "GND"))
 (segment (start 138.23 114.425) (end 148.68 114.425) (width 0.2) (layer "F.Cu") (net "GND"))
 (segment (start 173.58 101.575) (end 173.58 89.525) (width 0.2) (layer "F.Cu") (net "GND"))
 (segment (start 172.78 90.325) (end 162.33 90.325) (width 0.2) (layer "F.Cu") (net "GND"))
 (segment (start 148.68 114.425) (end 149.48 113.625) (width 0.2) (layer "F.Cu") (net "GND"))
 (segment (start 172.78 114.425) (end 173.58 113.625) (width 0.2) (layer "F.Cu") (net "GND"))
 (segment (start 138.23 90.325) (end 148.68 90.325) (width 0.2) (layer "F.Cu") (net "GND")))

